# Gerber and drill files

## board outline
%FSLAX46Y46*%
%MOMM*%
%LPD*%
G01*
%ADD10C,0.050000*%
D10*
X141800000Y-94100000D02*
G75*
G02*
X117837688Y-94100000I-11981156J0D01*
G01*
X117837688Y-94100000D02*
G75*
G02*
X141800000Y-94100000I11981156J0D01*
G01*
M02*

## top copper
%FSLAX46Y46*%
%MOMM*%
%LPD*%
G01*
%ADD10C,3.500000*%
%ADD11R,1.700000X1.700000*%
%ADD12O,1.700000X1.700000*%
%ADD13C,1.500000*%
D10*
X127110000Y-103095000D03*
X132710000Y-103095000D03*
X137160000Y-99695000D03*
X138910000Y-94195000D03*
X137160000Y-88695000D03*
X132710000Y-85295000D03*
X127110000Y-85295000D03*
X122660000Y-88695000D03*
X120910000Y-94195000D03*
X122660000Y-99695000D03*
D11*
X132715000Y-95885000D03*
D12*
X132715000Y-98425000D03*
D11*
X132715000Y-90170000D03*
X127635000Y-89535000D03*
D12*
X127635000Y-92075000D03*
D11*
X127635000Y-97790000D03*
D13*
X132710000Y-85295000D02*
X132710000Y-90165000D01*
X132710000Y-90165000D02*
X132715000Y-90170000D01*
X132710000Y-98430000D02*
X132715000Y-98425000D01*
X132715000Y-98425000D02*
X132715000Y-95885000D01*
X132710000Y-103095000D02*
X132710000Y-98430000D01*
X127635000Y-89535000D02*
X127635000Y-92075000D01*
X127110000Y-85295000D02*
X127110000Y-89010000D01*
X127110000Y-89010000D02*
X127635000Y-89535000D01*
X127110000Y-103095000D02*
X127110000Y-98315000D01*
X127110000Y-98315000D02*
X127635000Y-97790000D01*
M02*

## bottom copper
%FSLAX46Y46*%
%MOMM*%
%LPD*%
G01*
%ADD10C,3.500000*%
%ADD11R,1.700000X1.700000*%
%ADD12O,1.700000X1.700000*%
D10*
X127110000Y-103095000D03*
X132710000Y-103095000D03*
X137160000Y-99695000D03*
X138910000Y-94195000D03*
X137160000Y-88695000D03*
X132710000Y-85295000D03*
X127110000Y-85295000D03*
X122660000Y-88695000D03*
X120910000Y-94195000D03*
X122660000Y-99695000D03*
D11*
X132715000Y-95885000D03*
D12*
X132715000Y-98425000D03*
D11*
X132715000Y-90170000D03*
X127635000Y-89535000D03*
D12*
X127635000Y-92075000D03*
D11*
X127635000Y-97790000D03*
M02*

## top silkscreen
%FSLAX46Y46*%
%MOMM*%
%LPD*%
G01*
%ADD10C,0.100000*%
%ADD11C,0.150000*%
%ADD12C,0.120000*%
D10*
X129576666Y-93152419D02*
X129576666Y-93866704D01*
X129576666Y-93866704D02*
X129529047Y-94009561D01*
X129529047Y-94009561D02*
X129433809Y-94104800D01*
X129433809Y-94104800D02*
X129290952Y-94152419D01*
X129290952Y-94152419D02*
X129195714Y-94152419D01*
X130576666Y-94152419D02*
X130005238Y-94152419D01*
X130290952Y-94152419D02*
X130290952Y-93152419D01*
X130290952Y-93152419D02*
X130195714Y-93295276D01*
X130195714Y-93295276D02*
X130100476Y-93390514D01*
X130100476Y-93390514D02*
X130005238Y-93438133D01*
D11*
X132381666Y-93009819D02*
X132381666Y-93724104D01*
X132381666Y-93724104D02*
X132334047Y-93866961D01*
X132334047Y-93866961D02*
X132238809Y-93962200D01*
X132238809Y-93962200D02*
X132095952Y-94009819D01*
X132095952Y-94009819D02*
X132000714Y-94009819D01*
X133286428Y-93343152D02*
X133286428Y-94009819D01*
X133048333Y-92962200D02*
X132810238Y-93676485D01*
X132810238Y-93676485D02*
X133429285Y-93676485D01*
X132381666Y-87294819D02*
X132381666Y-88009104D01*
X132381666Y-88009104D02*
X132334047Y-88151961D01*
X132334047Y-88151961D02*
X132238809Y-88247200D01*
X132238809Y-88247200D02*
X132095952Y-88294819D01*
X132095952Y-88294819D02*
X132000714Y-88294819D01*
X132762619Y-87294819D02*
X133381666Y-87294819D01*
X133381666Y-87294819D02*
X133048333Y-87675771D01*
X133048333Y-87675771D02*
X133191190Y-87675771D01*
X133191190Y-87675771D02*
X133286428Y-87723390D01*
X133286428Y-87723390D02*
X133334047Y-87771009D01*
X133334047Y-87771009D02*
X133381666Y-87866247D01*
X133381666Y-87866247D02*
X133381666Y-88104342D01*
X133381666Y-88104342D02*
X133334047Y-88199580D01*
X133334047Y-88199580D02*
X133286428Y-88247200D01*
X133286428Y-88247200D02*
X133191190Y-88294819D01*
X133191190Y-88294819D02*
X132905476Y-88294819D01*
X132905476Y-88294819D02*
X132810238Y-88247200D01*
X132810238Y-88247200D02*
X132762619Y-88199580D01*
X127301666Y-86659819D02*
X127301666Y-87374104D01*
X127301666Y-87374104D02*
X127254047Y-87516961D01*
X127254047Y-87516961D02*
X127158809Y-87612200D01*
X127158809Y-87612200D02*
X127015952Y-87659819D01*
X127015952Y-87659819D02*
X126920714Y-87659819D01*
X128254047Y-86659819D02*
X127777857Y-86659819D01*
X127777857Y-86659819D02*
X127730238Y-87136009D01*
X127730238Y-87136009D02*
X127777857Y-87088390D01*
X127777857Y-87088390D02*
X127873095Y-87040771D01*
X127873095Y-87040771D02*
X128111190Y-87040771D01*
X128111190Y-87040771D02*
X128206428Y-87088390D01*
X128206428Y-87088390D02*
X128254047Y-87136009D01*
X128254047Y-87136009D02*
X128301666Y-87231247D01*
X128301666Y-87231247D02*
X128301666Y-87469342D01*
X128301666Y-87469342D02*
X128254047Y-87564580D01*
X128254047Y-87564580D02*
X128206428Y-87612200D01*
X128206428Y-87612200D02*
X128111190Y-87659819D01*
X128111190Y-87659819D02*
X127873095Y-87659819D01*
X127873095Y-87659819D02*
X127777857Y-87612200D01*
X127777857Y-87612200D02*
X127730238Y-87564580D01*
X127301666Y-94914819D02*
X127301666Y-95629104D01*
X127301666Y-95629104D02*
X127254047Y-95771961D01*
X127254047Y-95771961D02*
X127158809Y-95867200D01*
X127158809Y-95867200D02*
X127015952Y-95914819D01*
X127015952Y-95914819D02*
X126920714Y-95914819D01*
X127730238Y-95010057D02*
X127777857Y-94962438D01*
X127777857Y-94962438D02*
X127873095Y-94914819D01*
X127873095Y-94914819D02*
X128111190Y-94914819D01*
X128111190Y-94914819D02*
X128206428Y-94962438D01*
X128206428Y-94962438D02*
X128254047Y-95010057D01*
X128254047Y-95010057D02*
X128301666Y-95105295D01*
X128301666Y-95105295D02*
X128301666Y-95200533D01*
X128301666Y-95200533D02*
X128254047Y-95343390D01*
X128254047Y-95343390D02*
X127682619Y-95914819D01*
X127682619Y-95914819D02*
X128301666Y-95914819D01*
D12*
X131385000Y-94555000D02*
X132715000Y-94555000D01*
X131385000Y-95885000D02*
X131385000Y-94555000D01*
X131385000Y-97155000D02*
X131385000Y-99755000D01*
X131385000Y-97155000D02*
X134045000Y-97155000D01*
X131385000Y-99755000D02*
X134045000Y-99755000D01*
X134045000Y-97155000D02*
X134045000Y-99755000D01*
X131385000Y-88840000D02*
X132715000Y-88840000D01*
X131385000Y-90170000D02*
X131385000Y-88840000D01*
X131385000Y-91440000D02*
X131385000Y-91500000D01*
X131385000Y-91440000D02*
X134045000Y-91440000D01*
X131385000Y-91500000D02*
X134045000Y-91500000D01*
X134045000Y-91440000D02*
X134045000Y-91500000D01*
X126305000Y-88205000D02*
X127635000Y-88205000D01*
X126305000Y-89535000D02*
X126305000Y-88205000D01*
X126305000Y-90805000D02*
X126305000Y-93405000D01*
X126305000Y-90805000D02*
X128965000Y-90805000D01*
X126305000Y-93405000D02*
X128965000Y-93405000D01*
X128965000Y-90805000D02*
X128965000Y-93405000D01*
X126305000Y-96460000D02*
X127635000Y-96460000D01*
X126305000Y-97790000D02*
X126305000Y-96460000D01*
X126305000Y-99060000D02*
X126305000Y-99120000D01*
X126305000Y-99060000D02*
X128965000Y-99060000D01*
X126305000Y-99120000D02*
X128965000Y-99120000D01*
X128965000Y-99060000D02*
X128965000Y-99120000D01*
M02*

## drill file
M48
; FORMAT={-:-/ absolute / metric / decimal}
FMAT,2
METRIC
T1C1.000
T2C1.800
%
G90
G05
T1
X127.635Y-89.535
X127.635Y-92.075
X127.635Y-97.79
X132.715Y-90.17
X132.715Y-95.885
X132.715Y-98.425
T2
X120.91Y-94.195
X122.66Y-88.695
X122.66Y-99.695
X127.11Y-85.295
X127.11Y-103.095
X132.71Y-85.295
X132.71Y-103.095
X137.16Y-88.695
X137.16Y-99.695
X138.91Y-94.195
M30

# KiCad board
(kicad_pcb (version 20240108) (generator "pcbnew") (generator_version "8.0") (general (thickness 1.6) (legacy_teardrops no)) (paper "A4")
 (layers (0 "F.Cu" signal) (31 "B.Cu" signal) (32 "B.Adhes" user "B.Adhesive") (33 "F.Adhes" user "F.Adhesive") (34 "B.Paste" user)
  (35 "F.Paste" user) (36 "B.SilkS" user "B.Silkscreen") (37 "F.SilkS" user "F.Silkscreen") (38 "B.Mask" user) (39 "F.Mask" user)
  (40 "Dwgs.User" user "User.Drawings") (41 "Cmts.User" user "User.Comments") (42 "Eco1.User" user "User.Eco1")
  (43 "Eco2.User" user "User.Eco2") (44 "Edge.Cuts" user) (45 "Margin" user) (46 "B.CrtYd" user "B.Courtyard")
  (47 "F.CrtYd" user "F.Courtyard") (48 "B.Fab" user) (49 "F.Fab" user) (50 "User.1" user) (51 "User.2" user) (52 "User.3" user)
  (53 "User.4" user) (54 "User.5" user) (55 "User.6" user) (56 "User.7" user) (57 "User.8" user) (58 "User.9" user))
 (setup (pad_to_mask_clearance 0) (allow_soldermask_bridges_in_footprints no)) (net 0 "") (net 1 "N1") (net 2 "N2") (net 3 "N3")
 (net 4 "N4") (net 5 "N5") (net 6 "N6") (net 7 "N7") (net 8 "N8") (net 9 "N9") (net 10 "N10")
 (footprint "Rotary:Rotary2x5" (layer "F.Cu") (at 129.91 94.195)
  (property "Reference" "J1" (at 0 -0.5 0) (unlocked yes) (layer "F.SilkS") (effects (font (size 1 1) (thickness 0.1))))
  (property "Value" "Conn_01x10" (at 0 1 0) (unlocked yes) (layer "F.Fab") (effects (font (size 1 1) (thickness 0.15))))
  (pad "1" thru_hole circle (at -2.8 8.9) (size 3.5 3.5) (drill 1.8) (layers "*.Cu" "*.Mask") (remove_unused_layers no) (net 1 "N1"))
  (pad "2" thru_hole circle (at 2.8 8.9) (size 3.5 3.5) (drill 1.8) (layers "*.Cu" "*.Mask") (remove_unused_layers no) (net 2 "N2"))
  (pad "3" thru_hole circle (at 7.25 5.5) (size 3.5 3.5) (drill 1.8) (layers "*.Cu" "*.Mask") (remove_unused_layers no) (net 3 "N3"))
  (pad "4" thru_hole circle (at 9 0) (size 3.5 3.5) (drill 1.8) (layers "*.Cu" "*.Mask") (remove_unused_layers no) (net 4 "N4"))
  (pad "5" thru_hole circle (at 7.25 -5.5) (size 3.5 3.5) (drill 1.8) (layers "*.Cu" "*.Mask") (remove_unused_layers no) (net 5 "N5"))
  (pad "6" thru_hole circle (at 2.8 -8.9) (size 3.5 3.5) (drill 1.8) (layers "*.Cu" "*.Mask") (remove_unused_layers no) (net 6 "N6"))
  (pad "7" thru_hole circle (at -2.8 -8.9) (size 3.5 3.5) (drill 1.8) (layers "*.Cu" "*.Mask") (remove_unused_layers no) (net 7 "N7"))
  (pad "8" thru_hole circle (at -7.25 -5.5) (size 3.5 3.5) (drill 1.8) (layers "*.Cu" "*.Mask") (remove_unused_layers no) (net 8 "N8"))
  (pad "9" thru_hole circle (at -9 0) (size 3.5 3.5) (drill 1.8) (layers "*.Cu" "*.Mask") (remove_unused_layers no) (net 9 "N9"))
  (pad "10" thru_hole circle (at -7.25 5.5) (size 3.5 3.5) (drill 1.8) (layers "*.Cu" "*.Mask") (remove_unused_layers no) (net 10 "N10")))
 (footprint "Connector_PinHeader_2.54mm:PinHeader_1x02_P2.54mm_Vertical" (layer "F.Cu") (at 132.715 95.885)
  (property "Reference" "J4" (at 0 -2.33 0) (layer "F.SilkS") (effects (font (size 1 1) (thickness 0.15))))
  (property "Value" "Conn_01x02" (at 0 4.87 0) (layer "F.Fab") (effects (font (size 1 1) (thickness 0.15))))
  (fp_line (start -1.33 -1.33) (end 0 -1.33) (stroke (width 0.12) (type solid)) (layer "F.SilkS"))
  (fp_line (start -1.33 0) (end -1.33 -1.33) (stroke (width 0.12) (type solid)) (layer "F.SilkS"))
  (fp_line (start -1.33 1.27) (end -1.33 3.87) (stroke (width 0.12) (type solid)) (layer "F.SilkS"))
  (fp_line (start -1.33 1.27) (end 1.33 1.27) (stroke (width 0.12) (type solid)) (layer "F.SilkS"))
  (fp_line (start -1.33 3.87) (end 1.33 3.87) (stroke (width 0.12) (type solid)) (layer "F.SilkS"))
  (fp_line (start 1.33 1.27) (end 1.33 3.87) (stroke (width 0.12) (type solid)) (layer "F.SilkS"))
  (pad "1" thru_hole rect (at 0 0) (size 1.7 1.7) (drill 1) (layers "*.Cu" "*.Mask") (remove_unused_layers no) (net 2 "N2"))
  (pad "2" thru_hole oval (at 0 2.54) (size 1.7 1.7) (drill 1) (layers "*.Cu" "*.Mask") (remove_unused_layers no) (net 2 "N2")))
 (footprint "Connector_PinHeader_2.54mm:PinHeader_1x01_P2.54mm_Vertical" (layer "F.Cu") (at 132.715 90.17)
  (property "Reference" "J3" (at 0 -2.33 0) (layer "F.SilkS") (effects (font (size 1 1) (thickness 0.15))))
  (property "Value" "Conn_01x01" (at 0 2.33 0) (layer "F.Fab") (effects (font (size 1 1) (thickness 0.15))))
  (fp_line (start -1.33 -1.33) (end 0 -1.33) (stroke (width 0.12) (type solid)) (layer "F.SilkS"))
  (fp_line (start -1.33 0) (end -1.33 -1.33) (stroke (width 0.12) (type solid)) (layer "F.SilkS"))
  (fp_line (start -1.33 1.27) (end -1.33 1.33) (stroke (width 0.12) (type solid)) (layer "F.SilkS"))
  (fp_line (start -1.33 1.27) (end 1.33 1.27) (stroke (width 0.12) (type solid)) (layer "F.SilkS"))
  (fp_line (start -1.33 1.33) (end 1.33 1.33) (stroke (width 0.12) (type solid)) (layer "F.SilkS"))
  (fp_line (start 1.33 1.27) (end 1.33 1.33) (stroke (width 0.12) (type solid)) (layer "F.SilkS"))
  (pad "1" thru_hole rect (at 0 0) (size 1.7 1.7) (drill 1) (layers "*.Cu" "*.Mask") (remove_unused_layers no) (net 6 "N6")))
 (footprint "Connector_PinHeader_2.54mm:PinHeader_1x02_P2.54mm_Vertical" (layer "F.Cu") (at 127.635 89.535)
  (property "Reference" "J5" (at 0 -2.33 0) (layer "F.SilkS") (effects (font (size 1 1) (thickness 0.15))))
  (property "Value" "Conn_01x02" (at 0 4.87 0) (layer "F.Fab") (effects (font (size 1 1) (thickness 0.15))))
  (fp_line (start -1.33 -1.33) (end 0 -1.33) (stroke (width 0.12) (type solid)) (layer "F.SilkS"))
  (fp_line (start -1.33 0) (end -1.33 -1.33) (stroke (width 0.12) (type solid)) (layer "F.SilkS"))
  (fp_line (start -1.33 1.27) (end -1.33 3.87) (stroke (width 0.12) (type solid)) (layer "F.SilkS"))
  (fp_line (start -1.33 1.27) (end 1.33 1.27) (stroke (width 0.12) (type solid)) (layer "F.SilkS"))
  (fp_line (start -1.33 3.87) (end 1.33 3.87) (stroke (width 0.12) (type solid)) (layer "F.SilkS"))
  (fp_line (start 1.33 1.27) (end 1.33 3.87) (stroke (width 0.12) (type solid)) (layer "F.SilkS"))
  (pad "1" thru_hole rect (at 0 0) (size 1.7 1.7) (drill 1) (layers "*.Cu" "*.Mask") (remove_unused_layers no) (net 7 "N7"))
  (pad "2" thru_hole oval (at 0 2.54) (size 1.7 1.7) (drill 1) (layers "*.Cu" "*.Mask") (remove_unused_layers no) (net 7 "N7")))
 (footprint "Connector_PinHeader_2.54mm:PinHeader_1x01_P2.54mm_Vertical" (layer "F.Cu") (at 127.635 97.79)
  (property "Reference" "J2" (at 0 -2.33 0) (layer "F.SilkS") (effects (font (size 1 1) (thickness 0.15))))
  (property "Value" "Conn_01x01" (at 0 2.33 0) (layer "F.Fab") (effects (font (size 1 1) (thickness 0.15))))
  (fp_line (start -1.33 -1.33) (end 0 -1.33) (stroke (width 0.12) (type solid)) (layer "F.SilkS"))
  (fp_line (start -1.33 0) (end -1.33 -1.33) (stroke (width 0.12) (type solid)) (layer "F.SilkS"))
  (fp_line (start -1.33 1.27) (end -1.33 1.33) (stroke (width 0.12) (type solid)) (layer "F.SilkS"))
  (fp_line (start -1.33 1.27) (end 1.33 1.27) (stroke (width 0.12) (type solid)) (layer "F.SilkS"))
  (fp_line (start -1.33 1.33) (end 1.33 1.33) (stroke (width 0.12) (type solid)) (layer "F.SilkS"))
  (fp_line (start 1.33 1.27) (end 1.33 1.33) (stroke (width 0.12) (type solid)) (layer "F.SilkS"))
  (pad "1" thru_hole rect (at 0 0) (size 1.7 1.7) (drill 1) (layers "*.Cu" "*.Mask") (remove_unused_layers no) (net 1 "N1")))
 (gr_circle (center 129.818844 94.1) (end 139.978844 87.75) (stroke (width 0.05) (type default)) (fill none) (layer "Edge.Cuts"))
 (segment (start 132.71 85.295) (end 132.71 90.165) (width 1.5) (layer "F.Cu") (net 6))
 (segment (start 132.71 90.165) (end 132.715 90.17) (width 1.5) (layer "F.Cu") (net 6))
 (segment (start 132.71 98.43) (end 132.715 98.425) (width 1.5) (layer "F.Cu") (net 2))
 (segment (start 132.715 98.425) (end 132.715 95.885) (width 1.5) (layer "F.Cu") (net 2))
 (segment (start 132.71 103.095) (end 132.71 98.43) (width 1.5) (layer "F.Cu") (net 2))
 (segment (start 127.635 89.535) (end 127.635 92.075) (width 1.5) (layer "F.Cu") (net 7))
 (segment (start 127.11 85.295) (end 127.11 89.01) (width 1.5) (layer "F.Cu") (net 7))
 (segment (start 127.11 89.01) (end 127.635 89.535) (width 1.5) (layer "F.Cu") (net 7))
 (segment (start 127.11 103.095) (end 127.11 98.315) (width 1.5) (layer "F.Cu") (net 1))
 (segment (start 127.11 98.315) (end 127.635 97.79) (width 1.5) (layer "F.Cu") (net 1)))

